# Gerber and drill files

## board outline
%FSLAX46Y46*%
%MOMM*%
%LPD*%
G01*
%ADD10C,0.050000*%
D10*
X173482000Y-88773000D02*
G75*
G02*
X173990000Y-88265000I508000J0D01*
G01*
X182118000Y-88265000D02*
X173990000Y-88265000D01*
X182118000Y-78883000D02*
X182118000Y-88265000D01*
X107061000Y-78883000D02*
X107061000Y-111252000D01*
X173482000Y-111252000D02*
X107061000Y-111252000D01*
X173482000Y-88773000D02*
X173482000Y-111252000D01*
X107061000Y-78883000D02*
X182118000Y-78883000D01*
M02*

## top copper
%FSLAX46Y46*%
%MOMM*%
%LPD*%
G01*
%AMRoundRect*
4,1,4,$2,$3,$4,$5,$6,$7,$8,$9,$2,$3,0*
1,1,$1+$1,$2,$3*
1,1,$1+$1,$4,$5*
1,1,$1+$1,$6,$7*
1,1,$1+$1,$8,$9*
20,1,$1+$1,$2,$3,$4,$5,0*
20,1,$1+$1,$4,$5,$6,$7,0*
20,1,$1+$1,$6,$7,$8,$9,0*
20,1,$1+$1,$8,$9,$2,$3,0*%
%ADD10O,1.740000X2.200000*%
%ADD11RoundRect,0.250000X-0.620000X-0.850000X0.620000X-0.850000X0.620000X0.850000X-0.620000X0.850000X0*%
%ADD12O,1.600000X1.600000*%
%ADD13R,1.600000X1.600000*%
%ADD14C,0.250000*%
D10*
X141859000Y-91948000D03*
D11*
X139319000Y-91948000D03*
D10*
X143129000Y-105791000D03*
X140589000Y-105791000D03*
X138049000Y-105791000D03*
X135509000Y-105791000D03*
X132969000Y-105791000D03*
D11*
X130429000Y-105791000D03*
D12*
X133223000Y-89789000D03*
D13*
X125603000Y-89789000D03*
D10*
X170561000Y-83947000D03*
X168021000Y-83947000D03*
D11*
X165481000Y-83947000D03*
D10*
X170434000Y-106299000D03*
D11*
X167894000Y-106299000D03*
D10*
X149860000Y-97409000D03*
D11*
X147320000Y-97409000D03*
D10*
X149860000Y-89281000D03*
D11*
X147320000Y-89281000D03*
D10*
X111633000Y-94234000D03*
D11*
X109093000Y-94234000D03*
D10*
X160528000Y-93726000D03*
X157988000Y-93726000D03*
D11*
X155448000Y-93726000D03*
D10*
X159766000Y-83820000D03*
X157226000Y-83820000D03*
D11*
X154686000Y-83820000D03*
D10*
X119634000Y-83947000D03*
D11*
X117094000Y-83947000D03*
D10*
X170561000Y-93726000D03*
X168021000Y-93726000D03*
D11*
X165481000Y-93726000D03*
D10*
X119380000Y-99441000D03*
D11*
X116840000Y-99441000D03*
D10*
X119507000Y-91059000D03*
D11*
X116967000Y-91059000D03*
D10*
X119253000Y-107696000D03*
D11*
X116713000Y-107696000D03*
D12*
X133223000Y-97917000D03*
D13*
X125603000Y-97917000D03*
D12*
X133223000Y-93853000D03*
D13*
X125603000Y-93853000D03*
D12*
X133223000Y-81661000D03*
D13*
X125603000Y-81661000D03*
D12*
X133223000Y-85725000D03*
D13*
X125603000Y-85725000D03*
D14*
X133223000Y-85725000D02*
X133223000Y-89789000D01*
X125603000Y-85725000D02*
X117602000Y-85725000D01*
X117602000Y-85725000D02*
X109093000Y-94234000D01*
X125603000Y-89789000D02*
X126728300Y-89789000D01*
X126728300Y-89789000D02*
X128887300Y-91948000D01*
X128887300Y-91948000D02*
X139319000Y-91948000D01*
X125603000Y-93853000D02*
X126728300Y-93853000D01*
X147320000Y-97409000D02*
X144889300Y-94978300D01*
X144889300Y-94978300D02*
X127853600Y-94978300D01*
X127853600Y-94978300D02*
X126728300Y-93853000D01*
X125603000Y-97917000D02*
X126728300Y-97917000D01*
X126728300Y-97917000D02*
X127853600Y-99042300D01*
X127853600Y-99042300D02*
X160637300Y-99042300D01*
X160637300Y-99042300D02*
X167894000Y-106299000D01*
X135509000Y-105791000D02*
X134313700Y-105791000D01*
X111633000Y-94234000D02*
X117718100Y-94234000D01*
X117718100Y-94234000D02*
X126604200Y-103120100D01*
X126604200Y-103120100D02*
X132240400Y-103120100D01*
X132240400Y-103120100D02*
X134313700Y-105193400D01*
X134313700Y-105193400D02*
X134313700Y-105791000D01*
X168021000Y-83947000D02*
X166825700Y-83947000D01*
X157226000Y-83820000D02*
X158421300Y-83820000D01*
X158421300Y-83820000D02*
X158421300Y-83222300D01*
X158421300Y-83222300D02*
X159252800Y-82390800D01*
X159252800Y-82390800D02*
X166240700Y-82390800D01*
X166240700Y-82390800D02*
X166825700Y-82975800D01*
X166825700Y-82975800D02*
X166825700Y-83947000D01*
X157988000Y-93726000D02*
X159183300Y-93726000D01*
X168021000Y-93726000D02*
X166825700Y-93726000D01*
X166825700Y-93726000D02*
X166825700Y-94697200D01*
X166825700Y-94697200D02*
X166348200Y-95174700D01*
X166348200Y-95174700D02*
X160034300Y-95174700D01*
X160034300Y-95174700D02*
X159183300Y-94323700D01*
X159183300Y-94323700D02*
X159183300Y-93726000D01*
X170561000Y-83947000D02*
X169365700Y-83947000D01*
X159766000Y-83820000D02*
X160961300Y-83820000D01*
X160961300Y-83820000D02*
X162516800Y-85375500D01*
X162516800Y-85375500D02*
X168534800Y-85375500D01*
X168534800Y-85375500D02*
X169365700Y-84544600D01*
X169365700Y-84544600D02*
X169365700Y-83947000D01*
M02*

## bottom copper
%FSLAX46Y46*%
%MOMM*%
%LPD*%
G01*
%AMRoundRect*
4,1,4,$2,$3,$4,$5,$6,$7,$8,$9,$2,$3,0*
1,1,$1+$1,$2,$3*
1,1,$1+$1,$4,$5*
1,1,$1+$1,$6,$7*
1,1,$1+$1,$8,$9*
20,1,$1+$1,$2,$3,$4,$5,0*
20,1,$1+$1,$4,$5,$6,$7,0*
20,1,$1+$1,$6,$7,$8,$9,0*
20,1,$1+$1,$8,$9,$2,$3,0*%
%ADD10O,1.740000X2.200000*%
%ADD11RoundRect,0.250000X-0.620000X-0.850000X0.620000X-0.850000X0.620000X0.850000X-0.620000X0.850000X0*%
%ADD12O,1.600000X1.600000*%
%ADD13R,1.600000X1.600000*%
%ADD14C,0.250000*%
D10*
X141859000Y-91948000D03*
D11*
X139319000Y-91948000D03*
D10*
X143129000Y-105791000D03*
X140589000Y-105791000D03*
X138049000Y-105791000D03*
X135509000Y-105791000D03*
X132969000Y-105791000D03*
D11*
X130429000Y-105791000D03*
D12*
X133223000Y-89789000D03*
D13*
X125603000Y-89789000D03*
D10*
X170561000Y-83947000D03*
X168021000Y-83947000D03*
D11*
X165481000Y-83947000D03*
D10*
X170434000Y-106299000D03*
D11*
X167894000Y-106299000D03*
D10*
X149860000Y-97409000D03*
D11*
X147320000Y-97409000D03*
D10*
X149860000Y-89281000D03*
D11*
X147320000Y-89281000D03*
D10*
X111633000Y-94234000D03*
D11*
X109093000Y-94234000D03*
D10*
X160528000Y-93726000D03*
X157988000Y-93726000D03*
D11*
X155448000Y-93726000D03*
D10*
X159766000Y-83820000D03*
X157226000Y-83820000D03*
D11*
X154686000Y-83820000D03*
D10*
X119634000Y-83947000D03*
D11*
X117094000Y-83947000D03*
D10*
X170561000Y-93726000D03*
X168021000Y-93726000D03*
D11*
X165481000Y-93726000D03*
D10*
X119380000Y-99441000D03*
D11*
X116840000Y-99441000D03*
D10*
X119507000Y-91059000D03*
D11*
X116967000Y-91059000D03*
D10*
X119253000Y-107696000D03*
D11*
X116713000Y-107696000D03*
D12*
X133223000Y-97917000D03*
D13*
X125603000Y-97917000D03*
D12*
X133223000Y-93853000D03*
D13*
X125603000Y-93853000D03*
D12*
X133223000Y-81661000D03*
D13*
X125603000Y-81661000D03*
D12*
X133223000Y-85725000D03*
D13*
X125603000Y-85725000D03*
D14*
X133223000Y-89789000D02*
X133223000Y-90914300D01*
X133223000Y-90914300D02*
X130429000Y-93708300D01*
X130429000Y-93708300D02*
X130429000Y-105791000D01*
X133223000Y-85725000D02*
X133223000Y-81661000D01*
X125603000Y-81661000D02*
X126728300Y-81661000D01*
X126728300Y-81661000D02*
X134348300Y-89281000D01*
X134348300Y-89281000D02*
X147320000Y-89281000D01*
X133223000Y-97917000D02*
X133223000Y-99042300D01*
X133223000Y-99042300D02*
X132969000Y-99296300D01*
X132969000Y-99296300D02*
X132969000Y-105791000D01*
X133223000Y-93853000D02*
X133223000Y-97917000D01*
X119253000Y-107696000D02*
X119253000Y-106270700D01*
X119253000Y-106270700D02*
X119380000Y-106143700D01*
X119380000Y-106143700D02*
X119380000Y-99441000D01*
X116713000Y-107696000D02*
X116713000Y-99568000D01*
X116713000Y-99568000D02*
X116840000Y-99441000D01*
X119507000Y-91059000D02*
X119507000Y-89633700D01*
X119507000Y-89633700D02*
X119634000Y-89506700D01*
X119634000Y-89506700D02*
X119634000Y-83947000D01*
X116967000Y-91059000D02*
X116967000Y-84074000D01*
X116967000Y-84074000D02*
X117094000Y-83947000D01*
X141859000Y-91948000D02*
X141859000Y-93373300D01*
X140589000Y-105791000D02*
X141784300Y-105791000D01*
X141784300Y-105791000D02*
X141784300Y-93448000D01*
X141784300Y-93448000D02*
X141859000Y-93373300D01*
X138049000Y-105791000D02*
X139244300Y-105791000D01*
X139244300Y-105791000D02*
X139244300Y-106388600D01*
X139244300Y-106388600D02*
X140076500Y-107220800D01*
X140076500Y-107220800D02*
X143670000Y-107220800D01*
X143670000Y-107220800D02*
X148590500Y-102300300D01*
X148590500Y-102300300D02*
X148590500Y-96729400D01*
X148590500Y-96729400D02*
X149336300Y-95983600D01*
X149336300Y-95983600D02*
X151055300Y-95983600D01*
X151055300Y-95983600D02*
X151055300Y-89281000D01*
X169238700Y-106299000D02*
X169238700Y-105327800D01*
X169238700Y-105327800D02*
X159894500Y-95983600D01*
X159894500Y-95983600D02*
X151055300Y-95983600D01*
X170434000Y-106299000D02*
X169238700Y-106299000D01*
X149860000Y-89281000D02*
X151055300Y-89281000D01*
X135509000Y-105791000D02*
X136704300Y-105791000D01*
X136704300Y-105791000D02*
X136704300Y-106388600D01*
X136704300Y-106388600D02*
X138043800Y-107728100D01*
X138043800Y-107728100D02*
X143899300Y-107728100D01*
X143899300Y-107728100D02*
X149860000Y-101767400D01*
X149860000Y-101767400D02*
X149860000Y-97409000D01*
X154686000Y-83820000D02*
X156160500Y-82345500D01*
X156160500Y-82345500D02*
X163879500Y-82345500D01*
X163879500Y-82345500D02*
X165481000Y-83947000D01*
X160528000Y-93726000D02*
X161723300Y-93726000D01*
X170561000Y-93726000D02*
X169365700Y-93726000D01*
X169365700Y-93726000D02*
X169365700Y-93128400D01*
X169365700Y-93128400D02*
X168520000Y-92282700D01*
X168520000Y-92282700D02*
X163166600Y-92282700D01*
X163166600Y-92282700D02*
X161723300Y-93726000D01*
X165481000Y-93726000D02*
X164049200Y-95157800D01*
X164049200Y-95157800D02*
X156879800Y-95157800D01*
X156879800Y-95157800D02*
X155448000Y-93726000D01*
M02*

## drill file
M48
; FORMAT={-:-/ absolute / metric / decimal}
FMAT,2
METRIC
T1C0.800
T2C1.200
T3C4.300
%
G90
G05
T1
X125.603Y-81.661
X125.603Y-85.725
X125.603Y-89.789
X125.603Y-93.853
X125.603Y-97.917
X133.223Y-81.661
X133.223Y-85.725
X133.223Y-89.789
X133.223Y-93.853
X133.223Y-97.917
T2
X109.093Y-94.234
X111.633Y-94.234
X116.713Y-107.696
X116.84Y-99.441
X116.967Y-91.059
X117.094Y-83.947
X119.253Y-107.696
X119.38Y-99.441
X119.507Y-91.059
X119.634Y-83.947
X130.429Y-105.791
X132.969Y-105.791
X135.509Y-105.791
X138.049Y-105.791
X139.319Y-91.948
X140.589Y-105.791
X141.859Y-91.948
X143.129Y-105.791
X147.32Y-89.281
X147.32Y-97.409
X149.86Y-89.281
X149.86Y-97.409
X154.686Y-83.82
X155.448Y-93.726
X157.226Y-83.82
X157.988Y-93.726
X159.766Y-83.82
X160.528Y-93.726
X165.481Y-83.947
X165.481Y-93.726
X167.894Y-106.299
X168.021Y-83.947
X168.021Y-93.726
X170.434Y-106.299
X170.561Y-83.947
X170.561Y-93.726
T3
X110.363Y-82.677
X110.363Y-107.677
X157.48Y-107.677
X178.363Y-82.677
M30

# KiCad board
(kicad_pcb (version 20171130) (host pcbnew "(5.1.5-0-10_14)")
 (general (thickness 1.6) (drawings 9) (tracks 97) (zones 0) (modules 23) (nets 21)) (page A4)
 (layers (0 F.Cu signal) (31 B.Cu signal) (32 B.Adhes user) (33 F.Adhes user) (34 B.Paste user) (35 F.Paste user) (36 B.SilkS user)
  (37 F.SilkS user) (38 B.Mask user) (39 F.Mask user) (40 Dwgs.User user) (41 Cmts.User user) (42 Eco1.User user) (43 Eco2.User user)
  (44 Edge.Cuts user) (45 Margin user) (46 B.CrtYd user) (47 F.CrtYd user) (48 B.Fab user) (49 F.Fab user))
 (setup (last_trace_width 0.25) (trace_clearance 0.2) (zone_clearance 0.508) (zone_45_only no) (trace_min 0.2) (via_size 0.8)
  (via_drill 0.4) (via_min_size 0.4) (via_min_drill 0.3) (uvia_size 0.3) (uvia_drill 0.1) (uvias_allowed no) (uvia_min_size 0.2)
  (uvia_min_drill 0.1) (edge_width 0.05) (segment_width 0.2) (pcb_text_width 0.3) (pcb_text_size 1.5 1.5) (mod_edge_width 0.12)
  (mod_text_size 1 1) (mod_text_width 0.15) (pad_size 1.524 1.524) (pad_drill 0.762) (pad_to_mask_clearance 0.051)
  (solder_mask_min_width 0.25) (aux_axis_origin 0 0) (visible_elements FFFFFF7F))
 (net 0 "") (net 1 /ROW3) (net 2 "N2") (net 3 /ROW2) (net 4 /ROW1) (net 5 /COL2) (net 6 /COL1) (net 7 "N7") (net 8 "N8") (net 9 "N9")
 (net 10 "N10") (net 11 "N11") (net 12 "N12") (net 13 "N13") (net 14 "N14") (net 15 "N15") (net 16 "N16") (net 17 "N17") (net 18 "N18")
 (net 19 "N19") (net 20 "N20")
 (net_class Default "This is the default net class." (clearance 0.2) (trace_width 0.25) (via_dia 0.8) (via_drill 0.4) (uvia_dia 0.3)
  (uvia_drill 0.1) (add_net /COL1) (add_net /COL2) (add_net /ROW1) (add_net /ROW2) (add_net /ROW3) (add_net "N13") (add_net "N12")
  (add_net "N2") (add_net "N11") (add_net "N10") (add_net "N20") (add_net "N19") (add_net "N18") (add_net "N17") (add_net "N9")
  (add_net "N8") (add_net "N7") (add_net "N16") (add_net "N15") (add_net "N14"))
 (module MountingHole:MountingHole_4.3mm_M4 (layer F.Cu) (at 110.363 82.677)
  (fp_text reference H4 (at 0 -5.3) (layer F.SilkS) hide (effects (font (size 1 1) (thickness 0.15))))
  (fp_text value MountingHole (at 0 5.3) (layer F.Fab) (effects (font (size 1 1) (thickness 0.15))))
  (pad 1 np_thru_hole circle (at 0 0) (size 4.3 4.3) (drill 4.3) (layers *.Cu *.Mask)))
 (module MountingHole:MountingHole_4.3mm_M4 (layer F.Cu) (at 178.363 82.677)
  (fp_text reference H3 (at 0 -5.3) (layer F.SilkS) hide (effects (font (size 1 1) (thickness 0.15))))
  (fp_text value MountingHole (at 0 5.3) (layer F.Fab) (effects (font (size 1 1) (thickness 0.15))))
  (pad 1 np_thru_hole circle (at 0 0) (size 4.3 4.3) (drill 4.3) (layers *.Cu *.Mask)))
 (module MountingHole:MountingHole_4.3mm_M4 (layer F.Cu) (at 110.363 107.677)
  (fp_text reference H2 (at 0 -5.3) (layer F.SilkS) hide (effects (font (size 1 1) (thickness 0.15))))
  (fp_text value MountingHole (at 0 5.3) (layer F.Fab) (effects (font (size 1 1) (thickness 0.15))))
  (pad 1 np_thru_hole circle (at 0 0) (size 4.3 4.3) (drill 4.3) (layers *.Cu *.Mask)))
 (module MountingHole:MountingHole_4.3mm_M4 (layer F.Cu) (at 157.48 107.677)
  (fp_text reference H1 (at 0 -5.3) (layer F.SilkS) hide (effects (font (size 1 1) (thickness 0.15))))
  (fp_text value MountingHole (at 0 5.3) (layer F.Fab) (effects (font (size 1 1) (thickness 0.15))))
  (pad 1 np_thru_hole circle (at 0 0) (size 4.3 4.3) (drill 4.3) (layers *.Cu *.Mask)))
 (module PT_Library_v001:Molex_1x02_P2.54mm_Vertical (layer F.Cu) (at 139.319 91.948)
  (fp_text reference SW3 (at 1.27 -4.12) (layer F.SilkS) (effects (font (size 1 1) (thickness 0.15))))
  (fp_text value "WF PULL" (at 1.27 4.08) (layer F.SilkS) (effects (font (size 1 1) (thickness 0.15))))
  (pad 2 thru_hole oval (at 2.54 0) (size 1.74 2.2) (drill 1.2) (layers *.Cu *.Mask) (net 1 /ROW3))
  (pad 1 thru_hole roundrect (at 0 0) (size 1.74 2.2) (drill 1.2) (layers *.Cu *.Mask) (roundrect_rratio 0.143678) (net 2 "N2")))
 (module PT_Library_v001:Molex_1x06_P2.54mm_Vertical (layer F.Cu) (at 130.429 105.791)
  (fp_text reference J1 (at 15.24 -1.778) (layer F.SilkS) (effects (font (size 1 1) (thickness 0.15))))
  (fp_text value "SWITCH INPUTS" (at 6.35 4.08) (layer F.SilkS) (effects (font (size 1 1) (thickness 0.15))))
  (pad 6 thru_hole oval (at 12.7 0) (size 1.74 2.2) (drill 1.2) (layers *.Cu *.Mask))
  (pad 5 thru_hole oval (at 10.16 0) (size 1.74 2.2) (drill 1.2) (layers *.Cu *.Mask) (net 1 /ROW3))
  (pad 4 thru_hole oval (at 7.62 0) (size 1.74 2.2) (drill 1.2) (layers *.Cu *.Mask) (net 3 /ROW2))
  (pad 3 thru_hole oval (at 5.08 0) (size 1.74 2.2) (drill 1.2) (layers *.Cu *.Mask) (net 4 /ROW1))
  (pad 2 thru_hole oval (at 2.54 0) (size 1.74 2.2) (drill 1.2) (layers *.Cu *.Mask) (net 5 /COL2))
  (pad 1 thru_hole roundrect (at 0 0) (size 1.74 2.2) (drill 1.2) (layers *.Cu *.Mask) (roundrect_rratio 0.143678) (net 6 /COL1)))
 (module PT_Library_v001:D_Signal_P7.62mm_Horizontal (layer F.Cu) (at 125.603 89.789)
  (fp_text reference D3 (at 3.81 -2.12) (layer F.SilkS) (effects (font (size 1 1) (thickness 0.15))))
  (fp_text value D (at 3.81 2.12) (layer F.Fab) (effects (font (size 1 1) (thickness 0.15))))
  (pad 2 thru_hole oval (at 7.62 0) (size 1.6 1.6) (drill 0.8) (layers *.Cu *.Mask) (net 6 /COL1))
  (pad 1 thru_hole rect (at 0 0) (size 1.6 1.6) (drill 0.8) (layers *.Cu *.Mask) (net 2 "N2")))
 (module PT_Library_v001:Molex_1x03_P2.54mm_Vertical (layer F.Cu) (at 165.481 83.947)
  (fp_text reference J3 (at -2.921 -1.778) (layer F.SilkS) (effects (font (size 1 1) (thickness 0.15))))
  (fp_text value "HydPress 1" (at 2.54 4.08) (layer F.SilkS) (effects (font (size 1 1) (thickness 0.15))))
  (pad 3 thru_hole oval (at 5.08 0) (size 1.74 2.2) (drill 1.2) (layers *.Cu *.Mask) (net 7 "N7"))
  (pad 2 thru_hole oval (at 2.54 0) (size 1.74 2.2) (drill 1.2) (layers *.Cu *.Mask) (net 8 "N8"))
  (pad 1 thru_hole roundrect (at 0 0) (size 1.74 2.2) (drill 1.2) (layers *.Cu *.Mask) (roundrect_rratio 0.143678) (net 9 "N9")))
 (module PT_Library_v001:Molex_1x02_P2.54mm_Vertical (layer F.Cu) (at 167.894 106.299)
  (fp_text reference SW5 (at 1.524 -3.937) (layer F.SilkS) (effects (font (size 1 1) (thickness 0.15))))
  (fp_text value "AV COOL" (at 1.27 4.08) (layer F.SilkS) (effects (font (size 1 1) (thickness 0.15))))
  (pad 2 thru_hole oval (at 2.54 0) (size 1.74 2.2) (drill 1.2) (layers *.Cu *.Mask) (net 3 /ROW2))
  (pad 1 thru_hole roundrect (at 0 0) (size 1.74 2.2) (drill 1.2) (layers *.Cu *.Mask) (roundrect_rratio 0.143678) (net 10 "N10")))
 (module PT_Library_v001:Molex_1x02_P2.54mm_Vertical (layer F.Cu) (at 147.32 97.409)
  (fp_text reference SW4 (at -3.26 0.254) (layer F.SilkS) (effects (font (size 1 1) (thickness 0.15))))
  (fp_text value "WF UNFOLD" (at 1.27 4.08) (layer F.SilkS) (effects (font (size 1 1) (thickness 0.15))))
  (pad 2 thru_hole oval (at 2.54 0) (size 1.74 2.2) (drill 1.2) (layers *.Cu *.Mask) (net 4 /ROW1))
  (pad 1 thru_hole roundrect (at 0 0) (size 1.74 2.2) (drill 1.2) (layers *.Cu *.Mask) (roundrect_rratio 0.143678) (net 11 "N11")))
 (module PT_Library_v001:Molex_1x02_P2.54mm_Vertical (layer F.Cu) (at 147.32 89.281)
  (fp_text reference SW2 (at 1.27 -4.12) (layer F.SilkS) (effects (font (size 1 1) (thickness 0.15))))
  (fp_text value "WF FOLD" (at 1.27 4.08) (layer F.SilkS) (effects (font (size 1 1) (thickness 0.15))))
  (pad 2 thru_hole oval (at 2.54 0) (size 1.74 2.2) (drill 1.2) (layers *.Cu *.Mask) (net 3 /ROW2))
  (pad 1 thru_hole roundrect (at 0 0) (size 1.74 2.2) (drill 1.2) (layers *.Cu *.Mask) (roundrect_rratio 0.143678) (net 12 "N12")))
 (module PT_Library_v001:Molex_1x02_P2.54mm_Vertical (layer F.Cu) (at 109.093 94.234)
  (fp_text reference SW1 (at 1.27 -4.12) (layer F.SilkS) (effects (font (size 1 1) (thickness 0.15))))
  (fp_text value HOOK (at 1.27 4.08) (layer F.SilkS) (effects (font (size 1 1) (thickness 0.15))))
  (pad 2 thru_hole oval (at 2.54 0) (size 1.74 2.2) (drill 1.2) (layers *.Cu *.Mask) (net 4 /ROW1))
  (pad 1 thru_hole roundrect (at 0 0) (size 1.74 2.2) (drill 1.2) (layers *.Cu *.Mask) (roundrect_rratio 0.143678) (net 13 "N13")))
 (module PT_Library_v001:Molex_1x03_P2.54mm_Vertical (layer F.Cu) (at 155.448 93.726)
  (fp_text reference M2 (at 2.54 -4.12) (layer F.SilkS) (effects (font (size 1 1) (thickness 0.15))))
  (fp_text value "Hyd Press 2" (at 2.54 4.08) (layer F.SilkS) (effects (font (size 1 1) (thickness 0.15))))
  (pad 3 thru_hole oval (at 5.08 0) (size 1.74 2.2) (drill 1.2) (layers *.Cu *.Mask) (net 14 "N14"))
  (pad 2 thru_hole oval (at 2.54 0) (size 1.74 2.2) (drill 1.2) (layers *.Cu *.Mask) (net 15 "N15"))
  (pad 1 thru_hole roundrect (at 0 0) (size 1.74 2.2) (drill 1.2) (layers *.Cu *.Mask) (roundrect_rratio 0.143678) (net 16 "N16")))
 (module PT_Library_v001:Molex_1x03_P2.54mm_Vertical (layer F.Cu) (at 154.686 83.82)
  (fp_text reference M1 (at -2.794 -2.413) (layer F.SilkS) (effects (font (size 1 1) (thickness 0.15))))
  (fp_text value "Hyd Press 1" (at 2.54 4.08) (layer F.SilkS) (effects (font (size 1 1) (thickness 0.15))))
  (pad 3 thru_hole oval (at 5.08 0) (size 1.74 2.2) (drill 1.2) (layers *.Cu *.Mask) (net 7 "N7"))
  (pad 2 thru_hole oval (at 2.54 0) (size 1.74 2.2) (drill 1.2) (layers *.Cu *.Mask) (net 8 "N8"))
  (pad 1 thru_hole roundrect (at 0 0) (size 1.74 2.2) (drill 1.2) (layers *.Cu *.Mask) (roundrect_rratio 0.143678) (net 9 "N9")))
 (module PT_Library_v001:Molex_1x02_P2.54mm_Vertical (layer F.Cu) (at 117.094 83.947)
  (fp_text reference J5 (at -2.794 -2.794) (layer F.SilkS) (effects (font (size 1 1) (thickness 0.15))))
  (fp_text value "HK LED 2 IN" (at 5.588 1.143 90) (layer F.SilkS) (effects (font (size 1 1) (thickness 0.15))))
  (pad 2 thru_hole oval (at 2.54 0) (size 1.74 2.2) (drill 1.2) (layers *.Cu *.Mask) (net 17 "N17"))
  (pad 1 thru_hole roundrect (at 0 0) (size 1.74 2.2) (drill 1.2) (layers *.Cu *.Mask) (roundrect_rratio 0.143678) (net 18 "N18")))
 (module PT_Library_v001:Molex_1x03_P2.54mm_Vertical (layer F.Cu) (at 165.481 93.726)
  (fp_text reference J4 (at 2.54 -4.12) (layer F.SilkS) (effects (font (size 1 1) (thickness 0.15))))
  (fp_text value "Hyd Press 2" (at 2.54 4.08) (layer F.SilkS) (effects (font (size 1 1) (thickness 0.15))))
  (pad 3 thru_hole oval (at 5.08 0) (size 1.74 2.2) (drill 1.2) (layers *.Cu *.Mask) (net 14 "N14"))
  (pad 2 thru_hole oval (at 2.54 0) (size 1.74 2.2) (drill 1.2) (layers *.Cu *.Mask) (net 15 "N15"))
  (pad 1 thru_hole roundrect (at 0 0) (size 1.74 2.2) (drill 1.2) (layers *.Cu *.Mask) (roundrect_rratio 0.143678) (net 16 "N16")))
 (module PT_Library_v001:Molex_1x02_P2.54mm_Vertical (layer F.Cu) (at 116.84 99.441)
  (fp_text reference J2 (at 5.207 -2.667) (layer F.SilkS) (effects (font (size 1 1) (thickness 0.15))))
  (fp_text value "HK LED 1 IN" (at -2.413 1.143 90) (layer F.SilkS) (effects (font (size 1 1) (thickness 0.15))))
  (pad 2 thru_hole oval (at 2.54 0) (size 1.74 2.2) (drill 1.2) (layers *.Cu *.Mask) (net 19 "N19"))
  (pad 1 thru_hole roundrect (at 0 0) (size 1.74 2.2) (drill 1.2) (layers *.Cu *.Mask) (roundrect_rratio 0.143678) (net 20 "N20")))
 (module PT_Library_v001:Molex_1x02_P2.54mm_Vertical (layer F.Cu) (at 116.967 91.059)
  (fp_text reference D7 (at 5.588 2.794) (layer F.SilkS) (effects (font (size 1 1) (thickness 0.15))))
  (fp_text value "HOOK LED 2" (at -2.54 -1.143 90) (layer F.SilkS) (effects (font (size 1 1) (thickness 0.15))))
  (pad 2 thru_hole oval (at 2.54 0) (size 1.74 2.2) (drill 1.2) (layers *.Cu *.Mask) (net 17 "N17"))
  (pad 1 thru_hole roundrect (at 0 0) (size 1.74 2.2) (drill 1.2) (layers *.Cu *.Mask) (roundrect_rratio 0.143678) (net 18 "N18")))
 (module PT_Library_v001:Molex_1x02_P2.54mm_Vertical (layer F.Cu) (at 116.713 107.696)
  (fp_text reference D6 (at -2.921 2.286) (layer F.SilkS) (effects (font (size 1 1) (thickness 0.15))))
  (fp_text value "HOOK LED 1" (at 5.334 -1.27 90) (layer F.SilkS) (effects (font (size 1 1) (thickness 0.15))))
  (pad 2 thru_hole oval (at 2.54 0) (size 1.74 2.2) (drill 1.2) (layers *.Cu *.Mask) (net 19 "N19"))
  (pad 1 thru_hole roundrect (at 0 0) (size 1.74 2.2) (drill 1.2) (layers *.Cu *.Mask) (roundrect_rratio 0.143678) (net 20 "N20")))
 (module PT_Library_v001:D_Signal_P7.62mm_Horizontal (layer F.Cu) (at 125.603 97.917)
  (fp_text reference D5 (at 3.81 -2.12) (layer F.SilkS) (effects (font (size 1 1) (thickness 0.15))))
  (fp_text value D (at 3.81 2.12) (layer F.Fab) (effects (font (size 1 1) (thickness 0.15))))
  (pad 2 thru_hole oval (at 7.62 0) (size 1.6 1.6) (drill 0.8) (layers *.Cu *.Mask) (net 5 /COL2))
  (pad 1 thru_hole rect (at 0 0) (size 1.6 1.6) (drill 0.8) (layers *.Cu *.Mask) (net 10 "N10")))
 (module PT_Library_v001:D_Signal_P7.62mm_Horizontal (layer F.Cu) (at 125.603 93.853)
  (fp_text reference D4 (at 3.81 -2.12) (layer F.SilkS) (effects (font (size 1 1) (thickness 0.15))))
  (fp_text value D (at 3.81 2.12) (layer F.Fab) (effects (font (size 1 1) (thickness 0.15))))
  (pad 2 thru_hole oval (at 7.62 0) (size 1.6 1.6) (drill 0.8) (layers *.Cu *.Mask) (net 5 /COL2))
  (pad 1 thru_hole rect (at 0 0) (size 1.6 1.6) (drill 0.8) (layers *.Cu *.Mask) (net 11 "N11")))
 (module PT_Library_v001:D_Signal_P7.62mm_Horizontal (layer F.Cu) (at 125.603 81.661)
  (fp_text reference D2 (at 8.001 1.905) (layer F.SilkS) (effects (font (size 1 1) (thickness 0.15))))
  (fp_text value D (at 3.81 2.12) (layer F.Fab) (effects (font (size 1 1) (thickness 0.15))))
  (pad 2 thru_hole oval (at 7.62 0) (size 1.6 1.6) (drill 0.8) (layers *.Cu *.Mask) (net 6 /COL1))
  (pad 1 thru_hole rect (at 0 0) (size 1.6 1.6) (drill 0.8) (layers *.Cu *.Mask) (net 12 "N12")))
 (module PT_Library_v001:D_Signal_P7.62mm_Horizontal (layer F.Cu) (at 125.603 85.725)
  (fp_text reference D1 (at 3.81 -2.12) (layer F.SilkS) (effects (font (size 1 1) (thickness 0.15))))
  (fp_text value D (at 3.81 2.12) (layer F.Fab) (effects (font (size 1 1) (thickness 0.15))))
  (pad 2 thru_hole oval (at 7.62 0) (size 1.6 1.6) (drill 0.8) (layers *.Cu *.Mask) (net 6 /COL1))
  (pad 1 thru_hole rect (at 0 0) (size 1.6 1.6) (drill 0.8) (layers *.Cu *.Mask) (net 13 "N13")))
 (gr_arc (start 173.99 88.773) (end 173.99 88.265) (angle -90) (layer Edge.Cuts) (width 0.05))
 (gr_line (start 182.118 88.265) (end 173.99 88.265) (layer Edge.Cuts) (width 0.05))
 (gr_line (start 182.118 78.883) (end 182.118 88.265) (layer Edge.Cuts) (width 0.05))
 (gr_line (start 107.061 78.883) (end 107.061 111.252) (layer Edge.Cuts) (width 0.05))
 (gr_line (start 173.482 111.252) (end 107.061 111.252) (layer Edge.Cuts) (width 0.05))
 (gr_line (start 173.482 88.773) (end 173.482 111.252) (layer Edge.Cuts) (width 0.05))
 (gr_line (start 107.061 78.883) (end 182.118 78.883) (layer Edge.Cuts) (width 0.05))
 (segment (start 133.223 89.789) (end 133.223 90.9143) (width 0.25) (layer B.Cu) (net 6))
 (segment (start 133.223 90.9143) (end 130.429 93.7083) (width 0.25) (layer B.Cu) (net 6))
 (segment (start 130.429 93.7083) (end 130.429 105.791) (width 0.25) (layer B.Cu) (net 6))
 (segment (start 133.223 85.725) (end 133.223 89.789) (width 0.25) (layer F.Cu) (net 6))
 (segment (start 133.223 85.725) (end 133.223 81.661) (width 0.25) (layer B.Cu) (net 6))
 (segment (start 125.603 85.725) (end 117.602 85.725) (width 0.25) (layer F.Cu) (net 13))
 (segment (start 117.602 85.725) (end 109.093 94.234) (width 0.25) (layer F.Cu) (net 13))
 (segment (start 125.603 81.661) (end 126.7283 81.661) (width 0.25) (layer B.Cu) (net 12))
 (segment (start 126.7283 81.661) (end 134.3483 89.281) (width 0.25) (layer B.Cu) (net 12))
 (segment (start 134.3483 89.281) (end 147.32 89.281) (width 0.25) (layer B.Cu) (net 12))
 (segment (start 125.603 89.789) (end 126.7283 89.789) (width 0.25) (layer F.Cu) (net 2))
 (segment (start 126.7283 89.789) (end 128.8873 91.948) (width 0.25) (layer F.Cu) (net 2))
 (segment (start 128.8873 91.948) (end 139.319 91.948) (width 0.25) (layer F.Cu) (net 2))
 (segment (start 133.223 97.917) (end 133.223 99.0423) (width 0.25) (layer B.Cu) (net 5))
 (segment (start 133.223 99.0423) (end 132.969 99.2963) (width 0.25) (layer B.Cu) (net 5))
 (segment (start 132.969 99.2963) (end 132.969 105.791) (width 0.25) (layer B.Cu) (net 5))
 (segment (start 133.223 93.853) (end 133.223 97.917) (width 0.25) (layer B.Cu) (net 5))
 (segment (start 125.603 93.853) (end 126.7283 93.853) (width 0.25) (layer F.Cu) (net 11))
 (segment (start 147.32 97.409) (end 144.8893 94.9783) (width 0.25) (layer F.Cu) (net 11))
 (segment (start 144.8893 94.9783) (end 127.8536 94.9783) (width 0.25) (layer F.Cu) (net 11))
 (segment (start 127.8536 94.9783) (end 126.7283 93.853) (width 0.25) (layer F.Cu) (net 11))
 (segment (start 125.603 97.917) (end 126.7283 97.917) (width 0.25) (layer F.Cu) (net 10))
 (segment (start 126.7283 97.917) (end 127.8536 99.0423) (width 0.25) (layer F.Cu) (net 10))
 (segment (start 127.8536 99.0423) (end 160.6373 99.0423) (width 0.25) (layer F.Cu) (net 10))
 (segment (start 160.6373 99.0423) (end 167.894 106.299) (width 0.25) (layer F.Cu) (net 10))
 (segment (start 119.253 107.696) (end 119.253 106.2707) (width 0.25) (layer B.Cu) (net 19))
 (segment (start 119.253 106.2707) (end 119.38 106.1437) (width 0.25) (layer B.Cu) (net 19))
 (segment (start 119.38 106.1437) (end 119.38 99.441) (width 0.25) (layer B.Cu) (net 19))
 (segment (start 116.713 107.696) (end 116.713 99.568) (width 0.25) (layer B.Cu) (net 20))
 (segment (start 116.713 99.568) (end 116.84 99.441) (width 0.25) (layer B.Cu) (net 20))
 (segment (start 119.507 91.059) (end 119.507 89.6337) (width 0.25) (layer B.Cu) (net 17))
 (segment (start 119.507 89.6337) (end 119.634 89.5067) (width 0.25) (layer B.Cu) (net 17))
 (segment (start 119.634 89.5067) (end 119.634 83.947) (width 0.25) (layer B.Cu) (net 17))
 (segment (start 116.967 91.059) (end 116.967 84.074) (width 0.25) (layer B.Cu) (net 18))
 (segment (start 116.967 84.074) (end 117.094 83.947) (width 0.25) (layer B.Cu) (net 18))
 (segment (start 141.859 91.948) (end 141.859 93.3733) (width 0.25) (layer B.Cu) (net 1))
 (segment (start 140.589 105.791) (end 141.7843 105.791) (width 0.25) (layer B.Cu) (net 1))
 (segment (start 141.7843 105.791) (end 141.7843 93.448) (width 0.25) (layer B.Cu) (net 1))
 (segment (start 141.7843 93.448) (end 141.859 93.3733) (width 0.25) (layer B.Cu) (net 1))
 (segment (start 138.049 105.791) (end 139.2443 105.791) (width 0.25) (layer B.Cu) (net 3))
 (segment (start 139.2443 105.791) (end 139.2443 106.3886) (width 0.25) (layer B.Cu) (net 3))
 (segment (start 139.2443 106.3886) (end 140.0765 107.2208) (width 0.25) (layer B.Cu) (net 3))
 (segment (start 140.0765 107.2208) (end 143.67 107.2208) (width 0.25) (layer B.Cu) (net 3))
 (segment (start 143.67 107.2208) (end 148.5905 102.3003) (width 0.25) (layer B.Cu) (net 3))
 (segment (start 148.5905 102.3003) (end 148.5905 96.7294) (width 0.25) (layer B.Cu) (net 3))
 (segment (start 148.5905 96.7294) (end 149.3363 95.9836) (width 0.25) (layer B.Cu) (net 3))
 (segment (start 149.3363 95.9836) (end 151.0553 95.9836) (width 0.25) (layer B.Cu) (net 3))
 (segment (start 151.0553 95.9836) (end 151.0553 89.281) (width 0.25) (layer B.Cu) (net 3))
 (segment (start 169.2387 106.299) (end 169.2387 105.3278) (width 0.25) (layer B.Cu) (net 3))
 (segment (start 169.2387 105.3278) (end 159.8945 95.9836) (width 0.25) (layer B.Cu) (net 3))
 (segment (start 159.8945 95.9836) (end 151.0553 95.9836) (width 0.25) (layer B.Cu) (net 3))
 (segment (start 170.434 106.299) (end 169.2387 106.299) (width 0.25) (layer B.Cu) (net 3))
 (segment (start 149.86 89.281) (end 151.0553 89.281) (width 0.25) (layer B.Cu) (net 3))
 (segment (start 135.509 105.791) (end 134.3137 105.791) (width 0.25) (layer F.Cu) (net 4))
 (segment (start 111.633 94.234) (end 117.7181 94.234) (width 0.25) (layer F.Cu) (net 4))
 (segment (start 117.7181 94.234) (end 126.6042 103.1201) (width 0.25) (layer F.Cu) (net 4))
 (segment (start 126.6042 103.1201) (end 132.2404 103.1201) (width 0.25) (layer F.Cu) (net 4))
 (segment (start 132.2404 103.1201) (end 134.3137 105.1934) (width 0.25) (layer F.Cu) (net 4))
 (segment (start 134.3137 105.1934) (end 134.3137 105.791) (width 0.25) (layer F.Cu) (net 4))
 (segment (start 135.509 105.791) (end 136.7043 105.791) (width 0.25) (layer B.Cu) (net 4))
 (segment (start 136.7043 105.791) (end 136.7043 106.3886) (width 0.25) (layer B.Cu) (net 4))
 (segment (start 136.7043 106.3886) (end 138.0438 107.7281) (width 0.25) (layer B.Cu) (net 4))
 (segment (start 138.0438 107.7281) (end 143.8993 107.7281) (width 0.25) (layer B.Cu) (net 4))
 (segment (start 143.8993 107.7281) (end 149.86 101.7674) (width 0.25) (layer B.Cu) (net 4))
 (segment (start 149.86 101.7674) (end 149.86 97.409) (width 0.25) (layer B.Cu) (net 4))
 (segment (start 168.021 83.947) (end 166.8257 83.947) (width 0.25) (layer F.Cu) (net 8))
 (segment (start 157.226 83.82) (end 158.4213 83.82) (width 0.25) (layer F.Cu) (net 8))
 (segment (start 158.4213 83.82) (end 158.4213 83.2223) (width 0.25) (layer F.Cu) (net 8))
 (segment (start 158.4213 83.2223) (end 159.2528 82.3908) (width 0.25) (layer F.Cu) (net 8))
 (segment (start 159.2528 82.3908) (end 166.2407 82.3908) (width 0.25) (layer F.Cu) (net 8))
 (segment (start 166.2407 82.3908) (end 166.8257 82.9758) (width 0.25) (layer F.Cu) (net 8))
 (segment (start 166.8257 82.9758) (end 166.8257 83.947) (width 0.25) (layer F.Cu) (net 8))
 (segment (start 154.686 83.82) (end 156.1605 82.3455) (width 0.25) (layer B.Cu) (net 9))
 (segment (start 156.1605 82.3455) (end 163.8795 82.3455) (width 0.25) (layer B.Cu) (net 9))
 (segment (start 163.8795 82.3455) (end 165.481 83.947) (width 0.25) (layer B.Cu) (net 9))
 (segment (start 160.528 93.726) (end 161.7233 93.726) (width 0.25) (layer B.Cu) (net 14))
 (segment (start 170.561 93.726) (end 169.3657 93.726) (width 0.25) (layer B.Cu) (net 14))
 (segment (start 169.3657 93.726) (end 169.3657 93.1284) (width 0.25) (layer B.Cu) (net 14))
 (segment (start 169.3657 93.1284) (end 168.52 92.2827) (width 0.25) (layer B.Cu) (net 14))
 (segment (start 168.52 92.2827) (end 163.1666 92.2827) (width 0.25) (layer B.Cu) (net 14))
 (segment (start 163.1666 92.2827) (end 161.7233 93.726) (width 0.25) (layer B.Cu) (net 14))
 (segment (start 157.988 93.726) (end 159.1833 93.726) (width 0.25) (layer F.Cu) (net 15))
 (segment (start 168.021 93.726) (end 166.8257 93.726) (width 0.25) (layer F.Cu) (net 15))
 (segment (start 166.8257 93.726) (end 166.8257 94.6972) (width 0.25) (layer F.Cu) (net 15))
 (segment (start 166.8257 94.6972) (end 166.3482 95.1747) (width 0.25) (layer F.Cu) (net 15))
 (segment (start 166.3482 95.1747) (end 160.0343 95.1747) (width 0.25) (layer F.Cu) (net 15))
 (segment (start 160.0343 95.1747) (end 159.1833 94.3237) (width 0.25) (layer F.Cu) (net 15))
 (segment (start 159.1833 94.3237) (end 159.1833 93.726) (width 0.25) (layer F.Cu) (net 15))
 (segment (start 165.481 93.726) (end 164.0492 95.1578) (width 0.25) (layer B.Cu) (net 16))
 (segment (start 164.0492 95.1578) (end 156.8798 95.1578) (width 0.25) (layer B.Cu) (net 16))
 (segment (start 156.8798 95.1578) (end 155.448 93.726) (width 0.25) (layer B.Cu) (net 16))
 (segment (start 170.561 83.947) (end 169.3657 83.947) (width 0.25) (layer F.Cu) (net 7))
 (segment (start 159.766 83.82) (end 160.9613 83.82) (width 0.25) (layer F.Cu) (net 7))
 (segment (start 160.9613 83.82) (end 162.5168 85.3755) (width 0.25) (layer F.Cu) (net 7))
 (segment (start 162.5168 85.3755) (end 168.5348 85.3755) (width 0.25) (layer F.Cu) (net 7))
 (segment (start 168.5348 85.3755) (end 169.3657 84.5446) (width 0.25) (layer F.Cu) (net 7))
 (segment (start 169.3657 84.5446) (end 169.3657 83.947) (width 0.25) (layer F.Cu) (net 7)))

